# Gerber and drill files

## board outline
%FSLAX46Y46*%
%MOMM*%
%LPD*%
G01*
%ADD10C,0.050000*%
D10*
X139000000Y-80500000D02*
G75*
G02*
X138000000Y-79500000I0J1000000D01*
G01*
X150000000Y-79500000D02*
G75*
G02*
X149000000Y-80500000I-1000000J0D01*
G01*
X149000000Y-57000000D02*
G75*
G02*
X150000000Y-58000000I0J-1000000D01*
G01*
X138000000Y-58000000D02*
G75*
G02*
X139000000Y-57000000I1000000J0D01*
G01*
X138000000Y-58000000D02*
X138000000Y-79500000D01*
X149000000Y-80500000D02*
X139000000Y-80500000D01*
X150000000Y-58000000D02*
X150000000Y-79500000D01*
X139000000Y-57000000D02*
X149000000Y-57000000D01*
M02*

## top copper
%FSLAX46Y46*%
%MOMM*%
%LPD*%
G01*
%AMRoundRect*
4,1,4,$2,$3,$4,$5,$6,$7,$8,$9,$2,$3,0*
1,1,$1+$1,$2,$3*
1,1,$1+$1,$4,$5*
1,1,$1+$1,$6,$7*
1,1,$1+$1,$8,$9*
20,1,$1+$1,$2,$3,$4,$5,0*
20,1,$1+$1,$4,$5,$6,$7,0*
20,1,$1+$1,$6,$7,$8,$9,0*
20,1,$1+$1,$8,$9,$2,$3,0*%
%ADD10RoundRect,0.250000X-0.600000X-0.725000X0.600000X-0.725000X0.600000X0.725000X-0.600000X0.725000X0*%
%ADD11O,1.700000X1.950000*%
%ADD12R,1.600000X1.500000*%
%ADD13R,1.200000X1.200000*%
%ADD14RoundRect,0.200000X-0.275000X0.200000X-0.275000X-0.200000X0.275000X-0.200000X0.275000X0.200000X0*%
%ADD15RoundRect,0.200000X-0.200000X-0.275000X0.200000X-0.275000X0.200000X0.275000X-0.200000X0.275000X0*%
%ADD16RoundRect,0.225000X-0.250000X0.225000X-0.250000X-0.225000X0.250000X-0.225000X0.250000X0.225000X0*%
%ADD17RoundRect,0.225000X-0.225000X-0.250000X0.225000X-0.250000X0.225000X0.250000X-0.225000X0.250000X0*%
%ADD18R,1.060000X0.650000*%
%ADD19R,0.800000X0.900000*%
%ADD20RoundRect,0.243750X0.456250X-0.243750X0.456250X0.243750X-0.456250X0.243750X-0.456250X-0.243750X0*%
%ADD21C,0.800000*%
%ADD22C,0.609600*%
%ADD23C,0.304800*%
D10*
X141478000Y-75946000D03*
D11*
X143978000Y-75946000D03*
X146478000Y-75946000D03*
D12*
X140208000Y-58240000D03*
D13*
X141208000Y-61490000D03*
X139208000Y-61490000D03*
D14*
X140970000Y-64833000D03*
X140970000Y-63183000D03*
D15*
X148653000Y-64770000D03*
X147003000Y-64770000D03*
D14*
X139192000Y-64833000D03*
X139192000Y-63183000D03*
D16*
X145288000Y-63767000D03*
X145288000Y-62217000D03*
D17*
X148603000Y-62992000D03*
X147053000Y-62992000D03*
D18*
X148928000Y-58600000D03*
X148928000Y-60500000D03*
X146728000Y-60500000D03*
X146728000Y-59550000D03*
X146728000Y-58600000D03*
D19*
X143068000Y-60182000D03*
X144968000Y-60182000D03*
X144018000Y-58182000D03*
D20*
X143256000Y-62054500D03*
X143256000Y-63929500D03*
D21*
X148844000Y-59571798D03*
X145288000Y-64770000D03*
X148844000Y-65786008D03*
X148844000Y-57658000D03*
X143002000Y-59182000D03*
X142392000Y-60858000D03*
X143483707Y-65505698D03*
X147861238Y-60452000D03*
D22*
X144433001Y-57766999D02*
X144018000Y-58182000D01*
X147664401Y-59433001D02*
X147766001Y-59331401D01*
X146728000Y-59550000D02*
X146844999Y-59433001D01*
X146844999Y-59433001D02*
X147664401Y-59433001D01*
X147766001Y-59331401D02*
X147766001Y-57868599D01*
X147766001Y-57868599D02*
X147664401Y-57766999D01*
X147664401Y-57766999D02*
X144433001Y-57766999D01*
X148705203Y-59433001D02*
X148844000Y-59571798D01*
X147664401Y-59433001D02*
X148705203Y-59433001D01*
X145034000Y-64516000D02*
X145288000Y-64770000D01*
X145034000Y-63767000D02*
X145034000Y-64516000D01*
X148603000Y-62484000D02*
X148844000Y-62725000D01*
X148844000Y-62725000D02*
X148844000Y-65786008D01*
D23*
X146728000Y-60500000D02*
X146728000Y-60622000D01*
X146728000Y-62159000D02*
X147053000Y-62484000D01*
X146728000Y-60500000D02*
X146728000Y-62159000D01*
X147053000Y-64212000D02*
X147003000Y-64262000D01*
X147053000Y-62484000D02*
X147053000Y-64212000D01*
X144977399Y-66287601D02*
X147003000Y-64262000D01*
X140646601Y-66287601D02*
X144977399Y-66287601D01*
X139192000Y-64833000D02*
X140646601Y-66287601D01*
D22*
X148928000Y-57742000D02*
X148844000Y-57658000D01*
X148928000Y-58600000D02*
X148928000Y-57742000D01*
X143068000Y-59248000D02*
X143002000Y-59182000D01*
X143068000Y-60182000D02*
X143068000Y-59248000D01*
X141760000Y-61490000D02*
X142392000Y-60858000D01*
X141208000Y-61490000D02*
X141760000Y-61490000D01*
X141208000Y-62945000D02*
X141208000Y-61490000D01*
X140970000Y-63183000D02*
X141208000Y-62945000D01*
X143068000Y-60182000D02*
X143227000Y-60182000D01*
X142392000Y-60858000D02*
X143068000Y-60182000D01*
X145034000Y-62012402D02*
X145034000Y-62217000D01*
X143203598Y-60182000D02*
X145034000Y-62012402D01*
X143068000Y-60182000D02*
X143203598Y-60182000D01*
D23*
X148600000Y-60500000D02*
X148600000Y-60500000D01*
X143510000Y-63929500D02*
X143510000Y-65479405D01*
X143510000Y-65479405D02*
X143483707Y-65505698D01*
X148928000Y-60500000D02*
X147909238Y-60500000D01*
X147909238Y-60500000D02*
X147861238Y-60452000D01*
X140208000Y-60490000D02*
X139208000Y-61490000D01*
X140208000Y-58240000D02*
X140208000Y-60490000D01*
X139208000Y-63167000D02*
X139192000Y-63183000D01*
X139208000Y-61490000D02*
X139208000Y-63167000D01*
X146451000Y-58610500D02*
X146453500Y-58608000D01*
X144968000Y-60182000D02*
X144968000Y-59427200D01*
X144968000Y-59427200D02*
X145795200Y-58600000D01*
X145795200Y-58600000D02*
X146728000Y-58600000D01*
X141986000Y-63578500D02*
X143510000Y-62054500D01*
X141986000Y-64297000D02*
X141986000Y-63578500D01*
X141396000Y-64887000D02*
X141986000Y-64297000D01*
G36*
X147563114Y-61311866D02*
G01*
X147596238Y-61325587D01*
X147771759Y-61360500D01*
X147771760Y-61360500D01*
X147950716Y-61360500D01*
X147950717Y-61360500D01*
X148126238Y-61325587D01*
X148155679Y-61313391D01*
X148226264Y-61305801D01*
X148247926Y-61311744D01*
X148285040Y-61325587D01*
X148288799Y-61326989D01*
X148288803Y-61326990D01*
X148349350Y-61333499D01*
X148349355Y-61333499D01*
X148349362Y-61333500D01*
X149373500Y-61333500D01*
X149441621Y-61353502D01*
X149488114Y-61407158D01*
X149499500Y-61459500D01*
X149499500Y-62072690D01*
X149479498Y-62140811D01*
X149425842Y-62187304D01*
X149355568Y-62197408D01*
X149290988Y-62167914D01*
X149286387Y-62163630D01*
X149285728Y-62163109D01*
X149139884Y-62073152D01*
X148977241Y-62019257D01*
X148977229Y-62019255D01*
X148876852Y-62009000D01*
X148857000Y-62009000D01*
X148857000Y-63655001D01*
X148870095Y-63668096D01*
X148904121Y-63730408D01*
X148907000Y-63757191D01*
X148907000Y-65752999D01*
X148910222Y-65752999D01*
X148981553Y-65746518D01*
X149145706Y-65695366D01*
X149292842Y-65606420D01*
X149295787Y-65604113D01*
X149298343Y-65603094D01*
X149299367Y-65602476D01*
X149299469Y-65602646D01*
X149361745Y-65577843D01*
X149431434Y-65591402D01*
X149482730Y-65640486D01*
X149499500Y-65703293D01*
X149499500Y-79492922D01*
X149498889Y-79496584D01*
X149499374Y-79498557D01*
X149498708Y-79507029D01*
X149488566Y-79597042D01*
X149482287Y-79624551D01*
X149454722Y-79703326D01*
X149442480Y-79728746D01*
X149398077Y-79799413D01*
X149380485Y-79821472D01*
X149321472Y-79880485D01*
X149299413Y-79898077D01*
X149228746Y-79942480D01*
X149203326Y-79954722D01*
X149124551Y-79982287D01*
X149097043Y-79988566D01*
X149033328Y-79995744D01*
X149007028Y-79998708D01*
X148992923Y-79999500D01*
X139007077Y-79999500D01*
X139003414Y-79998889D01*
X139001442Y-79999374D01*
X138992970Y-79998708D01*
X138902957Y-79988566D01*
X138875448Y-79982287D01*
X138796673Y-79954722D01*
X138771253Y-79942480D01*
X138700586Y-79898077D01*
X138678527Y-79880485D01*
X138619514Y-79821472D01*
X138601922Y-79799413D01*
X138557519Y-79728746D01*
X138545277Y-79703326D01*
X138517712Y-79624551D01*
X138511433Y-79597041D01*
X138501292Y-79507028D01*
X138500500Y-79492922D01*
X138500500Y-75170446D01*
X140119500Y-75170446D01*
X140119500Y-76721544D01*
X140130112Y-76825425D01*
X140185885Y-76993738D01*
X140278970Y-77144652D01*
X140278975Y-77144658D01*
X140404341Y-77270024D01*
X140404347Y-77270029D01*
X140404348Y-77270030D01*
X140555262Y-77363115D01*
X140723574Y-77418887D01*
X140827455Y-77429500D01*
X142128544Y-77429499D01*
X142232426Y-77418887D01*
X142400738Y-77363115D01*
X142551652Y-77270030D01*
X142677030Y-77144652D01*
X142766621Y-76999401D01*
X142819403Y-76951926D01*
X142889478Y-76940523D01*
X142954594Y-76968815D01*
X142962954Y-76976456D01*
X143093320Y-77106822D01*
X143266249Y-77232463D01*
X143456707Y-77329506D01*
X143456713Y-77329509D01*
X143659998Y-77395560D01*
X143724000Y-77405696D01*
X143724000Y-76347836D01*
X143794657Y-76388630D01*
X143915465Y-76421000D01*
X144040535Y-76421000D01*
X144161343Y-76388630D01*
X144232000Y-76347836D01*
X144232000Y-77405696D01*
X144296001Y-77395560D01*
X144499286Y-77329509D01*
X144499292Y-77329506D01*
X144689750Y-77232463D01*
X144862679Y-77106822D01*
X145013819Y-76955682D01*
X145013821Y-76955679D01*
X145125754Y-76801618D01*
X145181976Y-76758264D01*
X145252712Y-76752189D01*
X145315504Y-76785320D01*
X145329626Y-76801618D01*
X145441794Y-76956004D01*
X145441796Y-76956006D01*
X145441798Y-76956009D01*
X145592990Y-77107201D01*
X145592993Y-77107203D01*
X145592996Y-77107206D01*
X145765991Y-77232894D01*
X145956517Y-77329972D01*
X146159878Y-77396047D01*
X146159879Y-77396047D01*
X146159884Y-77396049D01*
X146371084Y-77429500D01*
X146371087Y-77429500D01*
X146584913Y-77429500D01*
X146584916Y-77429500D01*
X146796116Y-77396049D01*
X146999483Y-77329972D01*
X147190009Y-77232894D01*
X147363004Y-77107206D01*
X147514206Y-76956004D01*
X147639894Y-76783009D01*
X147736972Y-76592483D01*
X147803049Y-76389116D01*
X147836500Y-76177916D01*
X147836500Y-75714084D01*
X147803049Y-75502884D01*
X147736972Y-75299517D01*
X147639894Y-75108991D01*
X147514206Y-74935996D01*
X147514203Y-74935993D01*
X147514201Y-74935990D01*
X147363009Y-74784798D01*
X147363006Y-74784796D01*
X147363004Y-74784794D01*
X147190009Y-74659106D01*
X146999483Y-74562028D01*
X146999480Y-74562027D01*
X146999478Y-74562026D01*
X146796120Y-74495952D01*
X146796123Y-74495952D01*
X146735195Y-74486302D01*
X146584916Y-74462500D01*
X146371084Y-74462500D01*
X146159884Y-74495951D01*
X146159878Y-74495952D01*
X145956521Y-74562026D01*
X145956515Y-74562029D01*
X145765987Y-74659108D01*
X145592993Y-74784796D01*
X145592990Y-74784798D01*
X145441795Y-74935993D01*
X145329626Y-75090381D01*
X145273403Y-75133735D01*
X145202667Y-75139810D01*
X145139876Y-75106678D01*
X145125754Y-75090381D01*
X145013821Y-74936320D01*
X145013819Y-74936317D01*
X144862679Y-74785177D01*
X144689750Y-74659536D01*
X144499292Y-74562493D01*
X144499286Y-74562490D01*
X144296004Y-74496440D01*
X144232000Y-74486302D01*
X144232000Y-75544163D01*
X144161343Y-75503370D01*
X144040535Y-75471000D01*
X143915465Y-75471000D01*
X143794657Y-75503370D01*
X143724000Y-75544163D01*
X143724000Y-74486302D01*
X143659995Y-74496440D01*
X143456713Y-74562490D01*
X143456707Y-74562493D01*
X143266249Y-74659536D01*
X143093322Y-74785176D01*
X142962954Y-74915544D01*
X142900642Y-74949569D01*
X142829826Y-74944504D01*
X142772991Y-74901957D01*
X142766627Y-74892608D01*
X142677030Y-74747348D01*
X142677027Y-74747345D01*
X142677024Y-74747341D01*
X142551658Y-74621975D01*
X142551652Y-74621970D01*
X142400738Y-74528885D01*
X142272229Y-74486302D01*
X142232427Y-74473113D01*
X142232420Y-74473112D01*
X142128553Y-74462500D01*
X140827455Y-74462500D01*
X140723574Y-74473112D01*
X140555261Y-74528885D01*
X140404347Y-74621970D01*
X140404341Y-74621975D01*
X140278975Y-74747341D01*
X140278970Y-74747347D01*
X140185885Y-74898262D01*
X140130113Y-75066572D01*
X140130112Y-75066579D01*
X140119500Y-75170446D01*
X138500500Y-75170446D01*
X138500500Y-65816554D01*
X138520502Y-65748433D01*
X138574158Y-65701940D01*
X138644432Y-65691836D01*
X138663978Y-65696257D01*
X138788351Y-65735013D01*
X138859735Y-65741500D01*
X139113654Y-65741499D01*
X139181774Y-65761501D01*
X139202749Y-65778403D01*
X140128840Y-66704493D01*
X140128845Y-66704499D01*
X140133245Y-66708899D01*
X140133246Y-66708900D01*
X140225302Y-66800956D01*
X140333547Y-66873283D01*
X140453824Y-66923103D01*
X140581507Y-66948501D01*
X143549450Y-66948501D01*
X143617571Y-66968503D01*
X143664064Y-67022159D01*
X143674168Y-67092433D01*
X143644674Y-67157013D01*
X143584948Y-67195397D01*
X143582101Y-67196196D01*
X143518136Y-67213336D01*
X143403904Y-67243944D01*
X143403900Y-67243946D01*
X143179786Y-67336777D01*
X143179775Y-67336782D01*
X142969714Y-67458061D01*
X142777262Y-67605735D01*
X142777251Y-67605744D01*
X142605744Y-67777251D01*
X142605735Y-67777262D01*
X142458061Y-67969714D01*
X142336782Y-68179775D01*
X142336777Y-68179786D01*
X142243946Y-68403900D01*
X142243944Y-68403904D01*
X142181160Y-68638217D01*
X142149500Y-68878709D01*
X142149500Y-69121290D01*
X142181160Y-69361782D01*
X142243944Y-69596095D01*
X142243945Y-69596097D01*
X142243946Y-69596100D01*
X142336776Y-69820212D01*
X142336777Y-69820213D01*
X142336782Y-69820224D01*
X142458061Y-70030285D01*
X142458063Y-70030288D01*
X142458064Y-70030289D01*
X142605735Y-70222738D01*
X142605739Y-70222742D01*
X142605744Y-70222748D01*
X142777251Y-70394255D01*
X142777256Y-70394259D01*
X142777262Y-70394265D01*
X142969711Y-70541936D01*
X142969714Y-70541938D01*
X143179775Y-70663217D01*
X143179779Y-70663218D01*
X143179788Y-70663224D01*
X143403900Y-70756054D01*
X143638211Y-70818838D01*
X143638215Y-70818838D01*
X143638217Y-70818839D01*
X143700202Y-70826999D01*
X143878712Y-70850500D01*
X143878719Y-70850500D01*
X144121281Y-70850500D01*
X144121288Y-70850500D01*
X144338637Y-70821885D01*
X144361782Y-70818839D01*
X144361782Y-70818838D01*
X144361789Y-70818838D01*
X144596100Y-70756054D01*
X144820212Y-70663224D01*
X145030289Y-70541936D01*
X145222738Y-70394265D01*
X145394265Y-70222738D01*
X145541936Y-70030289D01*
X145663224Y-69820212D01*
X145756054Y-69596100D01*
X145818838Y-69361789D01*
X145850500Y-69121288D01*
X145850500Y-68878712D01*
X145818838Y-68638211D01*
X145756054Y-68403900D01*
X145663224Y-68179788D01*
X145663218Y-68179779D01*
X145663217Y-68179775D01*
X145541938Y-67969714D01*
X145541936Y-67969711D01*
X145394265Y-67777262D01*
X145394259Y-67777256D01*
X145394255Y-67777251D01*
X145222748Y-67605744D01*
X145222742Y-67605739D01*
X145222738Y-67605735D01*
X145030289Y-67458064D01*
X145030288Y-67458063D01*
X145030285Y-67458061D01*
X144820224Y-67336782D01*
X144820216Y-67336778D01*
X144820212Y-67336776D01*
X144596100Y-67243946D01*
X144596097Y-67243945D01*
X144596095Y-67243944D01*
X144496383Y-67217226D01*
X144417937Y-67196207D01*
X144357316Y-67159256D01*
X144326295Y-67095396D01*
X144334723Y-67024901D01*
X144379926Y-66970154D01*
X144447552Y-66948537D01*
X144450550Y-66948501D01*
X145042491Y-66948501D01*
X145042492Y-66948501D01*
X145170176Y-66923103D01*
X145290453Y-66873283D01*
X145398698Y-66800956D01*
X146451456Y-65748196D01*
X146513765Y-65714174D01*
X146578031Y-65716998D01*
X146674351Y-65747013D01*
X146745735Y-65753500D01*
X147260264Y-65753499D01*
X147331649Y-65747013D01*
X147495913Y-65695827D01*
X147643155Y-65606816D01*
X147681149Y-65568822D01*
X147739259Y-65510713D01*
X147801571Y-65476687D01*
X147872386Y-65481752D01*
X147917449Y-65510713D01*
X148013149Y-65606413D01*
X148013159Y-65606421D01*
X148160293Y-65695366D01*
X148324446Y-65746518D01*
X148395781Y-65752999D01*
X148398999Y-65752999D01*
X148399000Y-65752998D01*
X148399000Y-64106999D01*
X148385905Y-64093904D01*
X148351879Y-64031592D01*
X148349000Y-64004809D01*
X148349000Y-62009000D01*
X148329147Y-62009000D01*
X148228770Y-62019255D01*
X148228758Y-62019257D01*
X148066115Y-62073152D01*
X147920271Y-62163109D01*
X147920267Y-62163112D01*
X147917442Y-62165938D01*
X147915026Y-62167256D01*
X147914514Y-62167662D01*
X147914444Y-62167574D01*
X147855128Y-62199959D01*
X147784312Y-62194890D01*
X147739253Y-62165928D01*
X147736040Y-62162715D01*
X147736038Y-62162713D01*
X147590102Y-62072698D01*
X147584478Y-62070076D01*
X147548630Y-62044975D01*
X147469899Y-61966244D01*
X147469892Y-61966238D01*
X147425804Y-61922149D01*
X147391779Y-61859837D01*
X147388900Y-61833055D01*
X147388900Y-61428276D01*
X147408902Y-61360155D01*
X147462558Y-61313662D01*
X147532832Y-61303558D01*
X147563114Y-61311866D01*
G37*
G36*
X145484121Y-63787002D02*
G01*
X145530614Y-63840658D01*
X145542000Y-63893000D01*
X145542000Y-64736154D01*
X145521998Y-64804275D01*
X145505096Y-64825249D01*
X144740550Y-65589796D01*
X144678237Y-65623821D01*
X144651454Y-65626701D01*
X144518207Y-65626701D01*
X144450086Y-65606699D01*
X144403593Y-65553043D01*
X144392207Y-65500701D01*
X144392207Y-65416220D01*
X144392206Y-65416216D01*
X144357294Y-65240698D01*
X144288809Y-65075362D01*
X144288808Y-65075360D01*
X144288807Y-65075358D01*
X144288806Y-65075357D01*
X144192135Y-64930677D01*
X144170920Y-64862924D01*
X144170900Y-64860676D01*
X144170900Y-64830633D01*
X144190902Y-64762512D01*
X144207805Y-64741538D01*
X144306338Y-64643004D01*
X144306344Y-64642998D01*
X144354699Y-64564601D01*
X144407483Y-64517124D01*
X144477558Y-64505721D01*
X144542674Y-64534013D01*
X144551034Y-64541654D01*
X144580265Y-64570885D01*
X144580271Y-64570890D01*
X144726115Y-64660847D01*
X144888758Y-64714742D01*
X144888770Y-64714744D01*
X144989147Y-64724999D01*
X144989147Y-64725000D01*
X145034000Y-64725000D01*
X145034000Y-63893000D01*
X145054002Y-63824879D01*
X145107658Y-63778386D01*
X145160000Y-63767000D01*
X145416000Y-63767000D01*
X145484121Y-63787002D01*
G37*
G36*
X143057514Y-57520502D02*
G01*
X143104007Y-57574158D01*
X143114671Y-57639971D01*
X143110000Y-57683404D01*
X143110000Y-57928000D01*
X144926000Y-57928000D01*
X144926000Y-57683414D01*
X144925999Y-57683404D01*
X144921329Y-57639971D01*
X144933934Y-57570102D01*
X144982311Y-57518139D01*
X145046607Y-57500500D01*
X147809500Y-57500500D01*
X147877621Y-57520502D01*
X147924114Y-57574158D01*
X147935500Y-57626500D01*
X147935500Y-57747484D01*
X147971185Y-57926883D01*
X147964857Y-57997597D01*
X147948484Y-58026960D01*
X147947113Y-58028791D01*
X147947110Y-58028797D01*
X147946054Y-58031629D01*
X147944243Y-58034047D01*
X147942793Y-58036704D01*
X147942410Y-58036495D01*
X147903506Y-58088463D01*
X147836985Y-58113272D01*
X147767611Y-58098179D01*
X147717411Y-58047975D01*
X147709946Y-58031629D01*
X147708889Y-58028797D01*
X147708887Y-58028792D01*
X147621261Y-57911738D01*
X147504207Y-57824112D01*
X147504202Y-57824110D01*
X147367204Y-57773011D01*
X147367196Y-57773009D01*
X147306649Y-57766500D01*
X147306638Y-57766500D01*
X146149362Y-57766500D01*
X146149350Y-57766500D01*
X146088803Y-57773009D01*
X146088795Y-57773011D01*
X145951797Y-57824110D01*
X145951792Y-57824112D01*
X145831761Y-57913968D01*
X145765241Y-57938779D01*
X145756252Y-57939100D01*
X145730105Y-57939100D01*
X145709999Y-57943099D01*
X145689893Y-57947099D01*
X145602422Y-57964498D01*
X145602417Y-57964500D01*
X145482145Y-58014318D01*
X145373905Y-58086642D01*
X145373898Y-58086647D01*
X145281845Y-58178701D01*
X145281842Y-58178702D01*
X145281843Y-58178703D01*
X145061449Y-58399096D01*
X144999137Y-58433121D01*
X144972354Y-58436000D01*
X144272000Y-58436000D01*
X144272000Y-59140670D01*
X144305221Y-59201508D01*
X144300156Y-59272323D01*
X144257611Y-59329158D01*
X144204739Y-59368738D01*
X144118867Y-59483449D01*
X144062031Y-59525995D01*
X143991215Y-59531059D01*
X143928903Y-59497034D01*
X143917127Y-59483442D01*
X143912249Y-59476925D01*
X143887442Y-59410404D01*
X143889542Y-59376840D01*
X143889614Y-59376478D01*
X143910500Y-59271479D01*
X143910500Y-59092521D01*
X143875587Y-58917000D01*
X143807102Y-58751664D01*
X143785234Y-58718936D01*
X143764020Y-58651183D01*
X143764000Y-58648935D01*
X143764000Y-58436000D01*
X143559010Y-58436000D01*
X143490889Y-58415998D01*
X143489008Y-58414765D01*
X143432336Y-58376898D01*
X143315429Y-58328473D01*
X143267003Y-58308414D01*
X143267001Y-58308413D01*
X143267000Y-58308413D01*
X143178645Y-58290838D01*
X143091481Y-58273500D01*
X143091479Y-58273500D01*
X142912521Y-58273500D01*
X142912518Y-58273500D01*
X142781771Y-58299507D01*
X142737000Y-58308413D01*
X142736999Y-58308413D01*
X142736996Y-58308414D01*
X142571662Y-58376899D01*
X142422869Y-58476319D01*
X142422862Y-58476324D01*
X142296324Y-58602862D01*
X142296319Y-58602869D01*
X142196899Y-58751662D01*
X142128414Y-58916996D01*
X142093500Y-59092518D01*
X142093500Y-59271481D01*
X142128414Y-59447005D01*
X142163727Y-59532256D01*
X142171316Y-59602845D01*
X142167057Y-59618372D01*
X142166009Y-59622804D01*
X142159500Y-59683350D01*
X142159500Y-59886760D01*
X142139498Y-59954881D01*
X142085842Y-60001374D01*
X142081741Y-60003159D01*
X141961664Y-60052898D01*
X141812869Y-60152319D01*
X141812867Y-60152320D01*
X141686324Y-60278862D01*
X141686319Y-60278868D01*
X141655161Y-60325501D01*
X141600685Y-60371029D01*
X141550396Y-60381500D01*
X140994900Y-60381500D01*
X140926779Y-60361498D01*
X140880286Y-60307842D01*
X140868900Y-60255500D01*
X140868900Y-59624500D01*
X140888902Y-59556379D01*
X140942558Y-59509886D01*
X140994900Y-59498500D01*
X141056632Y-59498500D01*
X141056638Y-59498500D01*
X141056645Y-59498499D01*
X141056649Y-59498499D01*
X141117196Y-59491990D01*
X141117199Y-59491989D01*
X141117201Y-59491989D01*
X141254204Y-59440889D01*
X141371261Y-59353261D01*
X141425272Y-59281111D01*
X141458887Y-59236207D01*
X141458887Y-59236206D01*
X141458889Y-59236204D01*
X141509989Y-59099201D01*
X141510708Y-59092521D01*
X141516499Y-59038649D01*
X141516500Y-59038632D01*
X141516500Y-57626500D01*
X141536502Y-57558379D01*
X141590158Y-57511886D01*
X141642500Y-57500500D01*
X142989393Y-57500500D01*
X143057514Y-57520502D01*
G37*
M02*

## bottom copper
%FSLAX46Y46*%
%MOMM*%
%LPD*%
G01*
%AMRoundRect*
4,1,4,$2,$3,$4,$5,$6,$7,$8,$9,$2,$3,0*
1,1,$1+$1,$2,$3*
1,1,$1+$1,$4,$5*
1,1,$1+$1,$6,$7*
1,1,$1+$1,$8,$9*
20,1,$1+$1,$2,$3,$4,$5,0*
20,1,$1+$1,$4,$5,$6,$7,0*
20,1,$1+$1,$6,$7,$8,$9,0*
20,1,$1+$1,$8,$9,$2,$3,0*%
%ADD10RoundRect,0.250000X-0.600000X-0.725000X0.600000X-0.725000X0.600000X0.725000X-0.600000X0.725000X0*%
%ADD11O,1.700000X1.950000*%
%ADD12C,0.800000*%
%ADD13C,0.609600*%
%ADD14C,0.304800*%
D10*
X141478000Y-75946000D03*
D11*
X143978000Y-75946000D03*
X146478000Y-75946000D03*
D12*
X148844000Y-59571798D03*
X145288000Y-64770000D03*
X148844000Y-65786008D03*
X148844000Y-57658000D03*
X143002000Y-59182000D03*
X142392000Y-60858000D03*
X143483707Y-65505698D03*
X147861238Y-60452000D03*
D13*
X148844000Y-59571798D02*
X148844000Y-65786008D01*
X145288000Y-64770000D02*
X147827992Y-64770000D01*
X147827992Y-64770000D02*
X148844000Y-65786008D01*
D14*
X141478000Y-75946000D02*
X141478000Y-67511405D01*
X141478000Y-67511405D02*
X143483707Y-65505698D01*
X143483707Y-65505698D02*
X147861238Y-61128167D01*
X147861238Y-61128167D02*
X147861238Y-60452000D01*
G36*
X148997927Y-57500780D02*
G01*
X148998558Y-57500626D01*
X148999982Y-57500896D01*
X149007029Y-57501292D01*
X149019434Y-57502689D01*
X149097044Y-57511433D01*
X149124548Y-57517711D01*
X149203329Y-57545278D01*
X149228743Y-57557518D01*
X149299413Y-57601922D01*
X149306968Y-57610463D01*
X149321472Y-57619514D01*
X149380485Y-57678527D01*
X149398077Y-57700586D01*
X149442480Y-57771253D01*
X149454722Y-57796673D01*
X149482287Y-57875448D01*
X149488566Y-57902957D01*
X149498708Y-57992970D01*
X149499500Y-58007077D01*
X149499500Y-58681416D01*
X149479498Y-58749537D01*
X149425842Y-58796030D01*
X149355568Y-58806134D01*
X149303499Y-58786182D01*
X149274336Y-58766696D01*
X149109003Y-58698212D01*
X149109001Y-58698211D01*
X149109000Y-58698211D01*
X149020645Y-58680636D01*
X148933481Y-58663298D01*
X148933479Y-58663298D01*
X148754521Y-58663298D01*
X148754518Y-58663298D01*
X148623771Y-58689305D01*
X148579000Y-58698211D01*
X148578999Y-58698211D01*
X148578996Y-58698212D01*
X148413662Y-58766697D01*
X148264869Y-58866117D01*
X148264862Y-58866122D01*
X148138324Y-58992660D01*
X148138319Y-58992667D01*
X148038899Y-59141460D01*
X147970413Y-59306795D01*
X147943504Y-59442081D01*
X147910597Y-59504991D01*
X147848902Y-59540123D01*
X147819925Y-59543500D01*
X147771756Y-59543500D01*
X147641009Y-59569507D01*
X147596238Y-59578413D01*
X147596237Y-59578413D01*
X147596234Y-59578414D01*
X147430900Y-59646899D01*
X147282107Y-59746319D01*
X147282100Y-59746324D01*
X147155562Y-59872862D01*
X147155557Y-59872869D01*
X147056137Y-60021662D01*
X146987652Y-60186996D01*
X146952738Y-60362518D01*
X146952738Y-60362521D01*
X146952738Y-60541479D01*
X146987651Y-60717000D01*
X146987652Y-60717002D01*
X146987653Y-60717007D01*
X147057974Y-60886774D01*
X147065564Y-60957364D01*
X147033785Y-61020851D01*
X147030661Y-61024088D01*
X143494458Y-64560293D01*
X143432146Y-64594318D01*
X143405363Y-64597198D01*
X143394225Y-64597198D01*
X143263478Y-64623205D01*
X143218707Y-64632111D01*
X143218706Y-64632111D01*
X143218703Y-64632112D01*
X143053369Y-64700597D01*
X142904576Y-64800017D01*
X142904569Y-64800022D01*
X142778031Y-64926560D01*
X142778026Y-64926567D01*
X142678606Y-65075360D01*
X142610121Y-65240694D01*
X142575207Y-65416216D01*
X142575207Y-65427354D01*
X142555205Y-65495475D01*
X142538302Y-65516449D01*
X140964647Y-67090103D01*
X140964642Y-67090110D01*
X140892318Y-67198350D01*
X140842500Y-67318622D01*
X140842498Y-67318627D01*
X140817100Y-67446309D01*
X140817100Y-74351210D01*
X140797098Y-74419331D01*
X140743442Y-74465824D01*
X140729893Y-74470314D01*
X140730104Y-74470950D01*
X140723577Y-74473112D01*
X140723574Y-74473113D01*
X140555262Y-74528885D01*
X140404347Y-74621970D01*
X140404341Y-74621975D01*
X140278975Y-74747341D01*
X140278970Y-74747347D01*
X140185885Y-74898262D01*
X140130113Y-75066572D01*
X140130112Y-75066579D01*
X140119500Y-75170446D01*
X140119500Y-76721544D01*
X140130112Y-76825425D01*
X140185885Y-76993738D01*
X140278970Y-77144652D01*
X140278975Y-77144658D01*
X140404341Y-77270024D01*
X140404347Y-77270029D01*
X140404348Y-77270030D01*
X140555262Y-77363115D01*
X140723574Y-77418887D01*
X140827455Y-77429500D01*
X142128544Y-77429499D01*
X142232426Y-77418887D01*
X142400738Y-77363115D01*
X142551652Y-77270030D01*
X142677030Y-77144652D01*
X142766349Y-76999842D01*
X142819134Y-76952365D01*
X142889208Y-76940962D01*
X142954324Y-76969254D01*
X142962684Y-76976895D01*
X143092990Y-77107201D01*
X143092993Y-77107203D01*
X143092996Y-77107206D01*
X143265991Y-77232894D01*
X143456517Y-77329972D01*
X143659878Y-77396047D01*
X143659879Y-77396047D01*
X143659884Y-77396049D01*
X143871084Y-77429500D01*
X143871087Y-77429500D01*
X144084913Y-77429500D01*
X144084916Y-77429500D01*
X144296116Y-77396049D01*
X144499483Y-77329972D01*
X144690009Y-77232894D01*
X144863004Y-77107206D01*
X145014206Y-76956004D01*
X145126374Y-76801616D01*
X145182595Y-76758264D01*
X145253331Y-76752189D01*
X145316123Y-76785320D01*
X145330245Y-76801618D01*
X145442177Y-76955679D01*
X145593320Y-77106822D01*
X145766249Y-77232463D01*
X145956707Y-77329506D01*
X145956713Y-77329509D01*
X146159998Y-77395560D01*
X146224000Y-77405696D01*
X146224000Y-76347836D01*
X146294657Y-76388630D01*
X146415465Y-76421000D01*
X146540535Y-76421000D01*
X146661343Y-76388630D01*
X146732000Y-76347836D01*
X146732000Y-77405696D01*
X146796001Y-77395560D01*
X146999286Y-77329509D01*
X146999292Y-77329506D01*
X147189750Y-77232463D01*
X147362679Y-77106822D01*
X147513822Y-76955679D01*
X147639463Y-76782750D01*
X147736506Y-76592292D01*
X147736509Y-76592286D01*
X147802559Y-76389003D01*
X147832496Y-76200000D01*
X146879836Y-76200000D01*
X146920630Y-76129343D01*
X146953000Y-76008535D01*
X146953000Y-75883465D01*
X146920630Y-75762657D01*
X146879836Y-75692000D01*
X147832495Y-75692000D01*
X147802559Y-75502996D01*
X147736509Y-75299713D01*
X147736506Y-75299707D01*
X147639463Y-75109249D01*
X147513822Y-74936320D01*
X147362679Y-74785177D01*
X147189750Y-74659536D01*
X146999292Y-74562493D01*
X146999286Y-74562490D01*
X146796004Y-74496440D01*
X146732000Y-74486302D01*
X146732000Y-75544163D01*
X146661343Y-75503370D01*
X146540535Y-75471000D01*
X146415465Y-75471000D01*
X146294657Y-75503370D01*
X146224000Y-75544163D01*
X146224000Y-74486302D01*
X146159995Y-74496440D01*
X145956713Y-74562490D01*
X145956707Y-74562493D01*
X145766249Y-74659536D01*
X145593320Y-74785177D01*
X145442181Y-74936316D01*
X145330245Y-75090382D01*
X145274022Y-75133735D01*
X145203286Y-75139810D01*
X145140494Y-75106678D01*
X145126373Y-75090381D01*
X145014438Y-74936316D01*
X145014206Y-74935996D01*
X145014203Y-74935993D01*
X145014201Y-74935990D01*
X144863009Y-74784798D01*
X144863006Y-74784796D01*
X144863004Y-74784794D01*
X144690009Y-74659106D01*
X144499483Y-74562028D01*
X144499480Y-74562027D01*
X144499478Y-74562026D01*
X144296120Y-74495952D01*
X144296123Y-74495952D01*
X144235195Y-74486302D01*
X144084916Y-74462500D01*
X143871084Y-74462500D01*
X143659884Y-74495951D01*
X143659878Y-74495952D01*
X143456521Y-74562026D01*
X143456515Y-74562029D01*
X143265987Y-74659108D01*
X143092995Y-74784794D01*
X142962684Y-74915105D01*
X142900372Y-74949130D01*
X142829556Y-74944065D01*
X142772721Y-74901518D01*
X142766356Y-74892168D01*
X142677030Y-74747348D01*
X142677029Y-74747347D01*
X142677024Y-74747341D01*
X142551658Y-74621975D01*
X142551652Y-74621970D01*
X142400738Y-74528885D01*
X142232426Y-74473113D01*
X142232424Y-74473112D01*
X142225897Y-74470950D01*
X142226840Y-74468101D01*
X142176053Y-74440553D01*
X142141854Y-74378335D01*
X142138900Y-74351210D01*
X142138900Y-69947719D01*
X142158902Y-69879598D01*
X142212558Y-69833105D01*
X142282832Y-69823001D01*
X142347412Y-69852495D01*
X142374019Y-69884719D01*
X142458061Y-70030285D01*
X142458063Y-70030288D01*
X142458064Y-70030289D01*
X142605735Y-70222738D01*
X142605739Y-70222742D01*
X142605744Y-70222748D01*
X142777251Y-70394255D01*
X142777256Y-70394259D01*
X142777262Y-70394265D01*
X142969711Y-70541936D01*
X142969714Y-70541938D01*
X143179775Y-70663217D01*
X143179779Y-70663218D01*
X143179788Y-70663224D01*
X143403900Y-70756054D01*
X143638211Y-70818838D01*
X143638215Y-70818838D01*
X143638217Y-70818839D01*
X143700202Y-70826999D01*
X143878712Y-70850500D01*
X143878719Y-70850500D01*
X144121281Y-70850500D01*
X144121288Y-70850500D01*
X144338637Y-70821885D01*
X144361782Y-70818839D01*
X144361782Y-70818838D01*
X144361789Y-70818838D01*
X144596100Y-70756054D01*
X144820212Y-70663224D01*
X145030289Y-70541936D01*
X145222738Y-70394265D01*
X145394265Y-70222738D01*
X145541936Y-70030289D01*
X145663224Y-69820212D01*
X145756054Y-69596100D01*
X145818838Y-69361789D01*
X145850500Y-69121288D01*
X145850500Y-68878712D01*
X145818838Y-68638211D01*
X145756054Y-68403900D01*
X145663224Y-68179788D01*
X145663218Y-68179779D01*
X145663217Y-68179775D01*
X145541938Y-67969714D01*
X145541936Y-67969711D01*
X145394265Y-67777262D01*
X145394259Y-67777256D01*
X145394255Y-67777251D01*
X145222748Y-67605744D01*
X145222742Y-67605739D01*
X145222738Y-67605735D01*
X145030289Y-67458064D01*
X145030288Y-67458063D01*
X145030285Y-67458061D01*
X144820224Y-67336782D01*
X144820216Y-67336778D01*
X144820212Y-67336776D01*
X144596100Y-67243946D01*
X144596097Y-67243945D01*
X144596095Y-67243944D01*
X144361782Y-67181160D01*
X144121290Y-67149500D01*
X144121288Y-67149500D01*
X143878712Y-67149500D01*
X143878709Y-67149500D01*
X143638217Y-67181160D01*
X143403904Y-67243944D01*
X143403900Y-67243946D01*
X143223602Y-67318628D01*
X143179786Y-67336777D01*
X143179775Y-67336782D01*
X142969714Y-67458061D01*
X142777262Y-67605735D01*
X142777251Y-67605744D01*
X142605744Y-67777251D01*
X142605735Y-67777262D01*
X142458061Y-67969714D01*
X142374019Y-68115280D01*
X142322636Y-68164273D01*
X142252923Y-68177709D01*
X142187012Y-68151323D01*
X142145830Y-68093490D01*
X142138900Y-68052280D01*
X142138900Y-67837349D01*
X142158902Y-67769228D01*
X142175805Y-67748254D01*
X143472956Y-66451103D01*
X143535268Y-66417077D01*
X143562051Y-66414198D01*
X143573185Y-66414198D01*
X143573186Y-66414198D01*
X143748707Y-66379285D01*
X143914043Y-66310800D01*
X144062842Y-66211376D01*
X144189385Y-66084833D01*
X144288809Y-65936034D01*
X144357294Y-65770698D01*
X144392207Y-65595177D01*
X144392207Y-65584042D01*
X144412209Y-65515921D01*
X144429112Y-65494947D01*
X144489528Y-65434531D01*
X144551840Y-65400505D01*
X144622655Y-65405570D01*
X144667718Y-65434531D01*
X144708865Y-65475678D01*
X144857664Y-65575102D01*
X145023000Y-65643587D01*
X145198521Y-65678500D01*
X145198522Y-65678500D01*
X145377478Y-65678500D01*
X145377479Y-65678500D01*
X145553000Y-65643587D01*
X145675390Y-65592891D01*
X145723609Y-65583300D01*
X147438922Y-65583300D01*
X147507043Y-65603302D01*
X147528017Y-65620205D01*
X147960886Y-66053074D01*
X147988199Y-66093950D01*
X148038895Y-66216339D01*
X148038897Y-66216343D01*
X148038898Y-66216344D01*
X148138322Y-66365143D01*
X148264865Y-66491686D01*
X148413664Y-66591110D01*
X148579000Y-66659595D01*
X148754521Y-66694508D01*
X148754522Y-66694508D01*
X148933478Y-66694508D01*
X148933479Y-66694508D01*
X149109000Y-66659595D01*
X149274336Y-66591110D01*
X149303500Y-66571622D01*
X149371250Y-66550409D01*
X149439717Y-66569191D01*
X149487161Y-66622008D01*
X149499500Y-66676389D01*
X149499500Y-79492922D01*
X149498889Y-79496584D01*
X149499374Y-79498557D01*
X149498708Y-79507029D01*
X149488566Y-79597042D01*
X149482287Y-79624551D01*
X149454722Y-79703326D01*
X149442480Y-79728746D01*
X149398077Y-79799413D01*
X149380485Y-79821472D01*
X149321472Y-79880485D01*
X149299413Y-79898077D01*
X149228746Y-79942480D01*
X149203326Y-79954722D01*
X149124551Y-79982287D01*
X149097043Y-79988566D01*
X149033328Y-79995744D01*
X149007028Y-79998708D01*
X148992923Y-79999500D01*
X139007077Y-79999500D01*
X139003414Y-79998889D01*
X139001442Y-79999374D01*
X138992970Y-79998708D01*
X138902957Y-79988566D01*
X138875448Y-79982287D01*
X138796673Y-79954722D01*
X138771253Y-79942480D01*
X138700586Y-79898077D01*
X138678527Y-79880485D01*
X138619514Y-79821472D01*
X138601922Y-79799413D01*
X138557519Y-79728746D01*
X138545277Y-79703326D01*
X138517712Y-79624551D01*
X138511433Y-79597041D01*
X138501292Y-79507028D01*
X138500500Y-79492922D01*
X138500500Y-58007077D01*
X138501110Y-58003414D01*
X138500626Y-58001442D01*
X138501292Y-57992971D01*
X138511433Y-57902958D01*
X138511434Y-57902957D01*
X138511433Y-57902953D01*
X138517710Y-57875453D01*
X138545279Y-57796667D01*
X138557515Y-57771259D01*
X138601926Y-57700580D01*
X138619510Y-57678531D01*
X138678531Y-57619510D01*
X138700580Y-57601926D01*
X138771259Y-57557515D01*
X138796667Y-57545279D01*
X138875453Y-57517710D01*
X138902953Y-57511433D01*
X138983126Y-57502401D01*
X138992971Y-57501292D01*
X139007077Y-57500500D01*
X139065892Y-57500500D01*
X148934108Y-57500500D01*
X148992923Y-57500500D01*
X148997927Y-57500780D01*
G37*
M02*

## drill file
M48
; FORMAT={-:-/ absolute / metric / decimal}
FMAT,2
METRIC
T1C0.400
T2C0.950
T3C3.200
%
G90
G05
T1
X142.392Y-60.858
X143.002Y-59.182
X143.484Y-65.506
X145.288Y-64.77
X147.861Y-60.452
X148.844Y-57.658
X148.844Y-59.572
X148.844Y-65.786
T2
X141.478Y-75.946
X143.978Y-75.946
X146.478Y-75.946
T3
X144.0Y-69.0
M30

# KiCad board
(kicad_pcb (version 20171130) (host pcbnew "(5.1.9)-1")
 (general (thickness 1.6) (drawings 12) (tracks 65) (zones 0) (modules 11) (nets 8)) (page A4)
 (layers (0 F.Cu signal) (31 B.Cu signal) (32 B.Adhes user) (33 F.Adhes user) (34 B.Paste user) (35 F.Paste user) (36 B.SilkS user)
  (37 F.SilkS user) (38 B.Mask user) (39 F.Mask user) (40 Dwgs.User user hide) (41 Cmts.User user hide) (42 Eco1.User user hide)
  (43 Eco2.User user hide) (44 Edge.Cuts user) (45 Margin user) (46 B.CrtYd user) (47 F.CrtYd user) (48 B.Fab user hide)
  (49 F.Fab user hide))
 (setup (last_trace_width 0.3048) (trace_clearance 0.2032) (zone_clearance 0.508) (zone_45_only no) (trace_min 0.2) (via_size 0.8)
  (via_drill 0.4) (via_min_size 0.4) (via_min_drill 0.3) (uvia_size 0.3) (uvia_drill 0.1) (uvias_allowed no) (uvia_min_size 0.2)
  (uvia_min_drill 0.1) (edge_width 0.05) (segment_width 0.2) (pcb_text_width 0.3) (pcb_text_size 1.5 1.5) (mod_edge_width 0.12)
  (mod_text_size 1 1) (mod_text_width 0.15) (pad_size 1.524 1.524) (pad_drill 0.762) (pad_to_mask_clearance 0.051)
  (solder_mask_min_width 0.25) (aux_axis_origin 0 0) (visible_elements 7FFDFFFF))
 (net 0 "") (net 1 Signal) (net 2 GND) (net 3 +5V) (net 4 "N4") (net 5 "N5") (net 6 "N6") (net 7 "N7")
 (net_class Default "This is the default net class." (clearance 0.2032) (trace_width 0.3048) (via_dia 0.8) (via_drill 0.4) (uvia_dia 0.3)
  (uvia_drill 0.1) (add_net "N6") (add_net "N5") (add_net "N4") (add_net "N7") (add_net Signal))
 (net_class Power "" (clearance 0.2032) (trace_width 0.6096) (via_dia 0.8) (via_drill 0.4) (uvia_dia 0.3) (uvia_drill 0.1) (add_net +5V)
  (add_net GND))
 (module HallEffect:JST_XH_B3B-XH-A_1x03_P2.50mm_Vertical (layer F.Cu) (at 141.478 75.946)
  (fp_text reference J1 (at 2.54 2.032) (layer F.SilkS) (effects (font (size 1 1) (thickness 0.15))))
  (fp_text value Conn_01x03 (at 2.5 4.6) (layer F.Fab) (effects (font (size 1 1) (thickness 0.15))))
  (pad 1 thru_hole roundrect (at 0 0) (size 1.7 1.95) (drill 0.95) (layers *.Cu *.Mask) (roundrect_rratio 0.147059) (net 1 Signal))
  (pad 2 thru_hole oval (at 2.5 0) (size 1.7 1.95) (drill 0.95) (layers *.Cu *.Mask) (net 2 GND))
  (pad 3 thru_hole oval (at 5 0) (size 1.7 1.95) (drill 0.95) (layers *.Cu *.Mask) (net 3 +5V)))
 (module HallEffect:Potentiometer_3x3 (layer F.Cu) (at 140.208 59.69 90)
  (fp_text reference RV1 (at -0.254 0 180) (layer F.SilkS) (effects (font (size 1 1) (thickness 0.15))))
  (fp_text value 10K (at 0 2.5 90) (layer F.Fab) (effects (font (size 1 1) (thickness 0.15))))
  (pad 2 smd rect (at 1.45 0 90) (size 1.5 1.6) (layers F.Cu F.Paste F.Mask) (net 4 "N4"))
  (pad 3 smd rect (at -1.8 1 90) (size 1.2 1.2) (layers F.Cu F.Paste F.Mask) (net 3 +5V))
  (pad 1 smd rect (at -1.8 -1 90) (size 1.2 1.2) (layers F.Cu F.Paste F.Mask) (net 4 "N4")))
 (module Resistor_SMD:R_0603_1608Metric (layer F.Cu) (at 140.97 64.008 270)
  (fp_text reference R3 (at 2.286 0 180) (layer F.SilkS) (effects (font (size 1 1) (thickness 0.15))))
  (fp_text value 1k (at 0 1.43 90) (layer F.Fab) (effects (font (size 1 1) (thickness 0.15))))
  (pad 2 smd roundrect (at 0.825 0 270) (size 0.8 0.95) (layers F.Cu F.Paste F.Mask) (roundrect_rratio 0.25) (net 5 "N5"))
  (pad 1 smd roundrect (at -0.825 0 270) (size 0.8 0.95) (layers F.Cu F.Paste F.Mask) (roundrect_rratio 0.25) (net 3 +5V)))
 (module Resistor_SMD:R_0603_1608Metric (layer F.Cu) (at 147.828 64.77)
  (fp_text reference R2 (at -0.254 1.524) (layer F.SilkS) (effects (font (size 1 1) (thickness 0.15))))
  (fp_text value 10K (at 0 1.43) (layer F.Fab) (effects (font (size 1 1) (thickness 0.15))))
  (pad 2 smd roundrect (at 0.825 0) (size 0.8 0.95) (layers F.Cu F.Paste F.Mask) (roundrect_rratio 0.25) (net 2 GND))
  (pad 1 smd roundrect (at -0.825 0) (size 0.8 0.95) (layers F.Cu F.Paste F.Mask) (roundrect_rratio 0.25) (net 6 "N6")))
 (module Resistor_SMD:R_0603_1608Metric (layer F.Cu) (at 139.192 64.008 270)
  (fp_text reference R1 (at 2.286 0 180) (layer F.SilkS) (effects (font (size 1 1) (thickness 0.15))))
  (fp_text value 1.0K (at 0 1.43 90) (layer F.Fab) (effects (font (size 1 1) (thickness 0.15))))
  (pad 2 smd roundrect (at 0.825 0 270) (size 0.8 0.95) (layers F.Cu F.Paste F.Mask) (roundrect_rratio 0.25) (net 6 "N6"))
  (pad 1 smd roundrect (at -0.825 0 270) (size 0.8 0.95) (layers F.Cu F.Paste F.Mask) (roundrect_rratio 0.25) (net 4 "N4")))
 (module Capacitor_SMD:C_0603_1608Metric (layer F.Cu) (at 145.288 62.992 270)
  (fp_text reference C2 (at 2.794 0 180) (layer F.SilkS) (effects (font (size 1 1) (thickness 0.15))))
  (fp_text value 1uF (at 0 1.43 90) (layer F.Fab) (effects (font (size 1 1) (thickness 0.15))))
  (pad 2 smd roundrect (at 0.775 0 270) (size 0.9 0.95) (layers F.Cu F.Paste F.Mask) (roundrect_rratio 0.25) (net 2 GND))
  (pad 1 smd roundrect (at -0.775 0 270) (size 0.9 0.95) (layers F.Cu F.Paste F.Mask) (roundrect_rratio 0.25) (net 3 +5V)))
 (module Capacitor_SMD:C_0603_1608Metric (layer F.Cu) (at 147.828 62.992)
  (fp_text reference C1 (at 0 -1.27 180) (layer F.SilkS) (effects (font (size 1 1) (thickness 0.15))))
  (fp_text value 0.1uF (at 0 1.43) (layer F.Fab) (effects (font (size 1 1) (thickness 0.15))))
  (pad 2 smd roundrect (at 0.775 0) (size 0.9 0.95) (layers F.Cu F.Paste F.Mask) (roundrect_rratio 0.25) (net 2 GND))
  (pad 1 smd roundrect (at -0.775 0) (size 0.9 0.95) (layers F.Cu F.Paste F.Mask) (roundrect_rratio 0.25) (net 6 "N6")))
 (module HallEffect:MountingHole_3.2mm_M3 (layer F.Cu) (at 144 69)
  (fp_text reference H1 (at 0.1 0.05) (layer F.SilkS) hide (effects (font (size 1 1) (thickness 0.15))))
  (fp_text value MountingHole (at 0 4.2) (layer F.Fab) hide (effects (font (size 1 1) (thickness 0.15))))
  (pad 1 np_thru_hole circle (at 0 0) (size 3.2 3.2) (drill 3.2) (layers *.Cu *.Mask)))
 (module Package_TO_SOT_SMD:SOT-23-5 (layer F.Cu) (at 147.828 59.55)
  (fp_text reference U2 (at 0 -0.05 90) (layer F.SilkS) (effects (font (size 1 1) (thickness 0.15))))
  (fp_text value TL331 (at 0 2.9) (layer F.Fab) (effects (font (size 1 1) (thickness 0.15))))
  (pad 5 smd rect (at 1.1 -0.95) (size 1.06 0.65) (layers F.Cu F.Paste F.Mask) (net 3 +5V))
  (pad 4 smd rect (at 1.1 0.95) (size 1.06 0.65) (layers F.Cu F.Paste F.Mask) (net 1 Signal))
  (pad 3 smd rect (at -1.1 0.95) (size 1.06 0.65) (layers F.Cu F.Paste F.Mask) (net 6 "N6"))
  (pad 2 smd rect (at -1.1 0) (size 1.06 0.65) (layers F.Cu F.Paste F.Mask) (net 2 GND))
  (pad 1 smd rect (at -1.1 -0.95) (size 1.06 0.65) (layers F.Cu F.Paste F.Mask) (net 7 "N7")))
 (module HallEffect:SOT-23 (layer F.Cu) (at 144.018 59.182 90)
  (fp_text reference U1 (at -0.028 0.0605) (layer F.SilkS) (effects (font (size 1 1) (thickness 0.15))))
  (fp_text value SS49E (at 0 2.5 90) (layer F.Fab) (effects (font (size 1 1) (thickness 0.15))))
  (pad 1 smd rect (at -1 -0.95 90) (size 0.9 0.8) (layers F.Cu F.Paste F.Mask) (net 3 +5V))
  (pad 2 smd rect (at -1 0.95 90) (size 0.9 0.8) (layers F.Cu F.Paste F.Mask) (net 7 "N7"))
  (pad 3 smd rect (at 1 0 90) (size 0.9 0.8) (layers F.Cu F.Paste F.Mask) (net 2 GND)))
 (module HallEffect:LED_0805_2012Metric (layer F.Cu) (at 143.256 62.992 90)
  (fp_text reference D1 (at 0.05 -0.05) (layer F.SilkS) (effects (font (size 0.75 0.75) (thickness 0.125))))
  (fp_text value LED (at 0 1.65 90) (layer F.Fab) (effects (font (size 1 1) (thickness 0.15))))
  (pad 2 smd roundrect (at 0.9375 0 90) (size 0.975 1.4) (layers F.Cu F.Paste F.Mask) (roundrect_rratio 0.25) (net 5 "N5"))
  (pad 1 smd roundrect (at -0.9375 0 90) (size 0.975 1.4) (layers F.Cu F.Paste F.Mask) (roundrect_rratio 0.25) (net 1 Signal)))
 (gr_arc (start 139 79.5) (end 138 79.5) (angle -90) (layer Edge.Cuts) (width 0.05))
 (gr_arc (start 149 79.5) (end 149 80.5) (angle -90) (layer Edge.Cuts) (width 0.05))
 (gr_arc (start 149 58) (end 150 58) (angle -90) (layer Edge.Cuts) (width 0.05))
 (gr_arc (start 139 58) (end 139 57) (angle -90) (layer Edge.Cuts) (width 0.05))
 (gr_line (start 138 58) (end 138 79.5) (layer Edge.Cuts) (width 0.05))
 (gr_line (start 149 80.5) (end 139 80.5) (layer Edge.Cuts) (width 0.05))
 (gr_line (start 150 58) (end 150 79.5) (layer Edge.Cuts) (width 0.05))
 (gr_line (start 139 57) (end 149 57) (layer Edge.Cuts) (width 0.05))
 (segment (start 144.433001 57.766999) (end 144.018 58.182) (width 0.6096) (layer F.Cu) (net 2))
 (segment (start 147.664401 59.433001) (end 147.766001 59.331401) (width 0.6096) (layer F.Cu) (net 2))
 (segment (start 146.728 59.55) (end 146.844999 59.433001) (width 0.6096) (layer F.Cu) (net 2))
 (segment (start 146.844999 59.433001) (end 147.664401 59.433001) (width 0.6096) (layer F.Cu) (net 2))
 (segment (start 147.766001 59.331401) (end 147.766001 57.868599) (width 0.6096) (layer F.Cu) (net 2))
 (segment (start 147.766001 57.868599) (end 147.664401 57.766999) (width 0.6096) (layer F.Cu) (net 2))
 (segment (start 147.664401 57.766999) (end 144.433001 57.766999) (width 0.6096) (layer F.Cu) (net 2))
 (via (at 148.844 59.571798) (size 0.8) (drill 0.4) (layers F.Cu B.Cu) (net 2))
 (segment (start 148.705203 59.433001) (end 148.844 59.571798) (width 0.6096) (layer F.Cu) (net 2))
 (segment (start 147.664401 59.433001) (end 148.705203 59.433001) (width 0.6096) (layer F.Cu) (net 2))
 (via (at 145.288 64.77) (size 0.8) (drill 0.4) (layers F.Cu B.Cu) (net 2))
 (segment (start 145.034 64.516) (end 145.288 64.77) (width 0.6096) (layer F.Cu) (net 2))
 (segment (start 145.034 63.767) (end 145.034 64.516) (width 0.6096) (layer F.Cu) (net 2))
 (segment (start 148.844 59.571798) (end 148.844 65.786008) (width 0.6096) (layer B.Cu) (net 2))
 (via (at 148.844 65.786008) (size 0.8) (drill 0.4) (layers F.Cu B.Cu) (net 2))
 (segment (start 148.603 62.484) (end 148.844 62.725) (width 0.6096) (layer F.Cu) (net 2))
 (segment (start 148.844 62.725) (end 148.844 65.786008) (width 0.6096) (layer F.Cu) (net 2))
 (segment (start 145.288 64.77) (end 147.827992 64.77) (width 0.6096) (layer B.Cu) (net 2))
 (segment (start 147.827992 64.77) (end 148.844 65.786008) (width 0.6096) (layer B.Cu) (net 2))
 (segment (start 146.728 60.5) (end 146.728 60.622) (width 0.3048) (layer F.Cu) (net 6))
 (segment (start 146.728 62.159) (end 147.053 62.484) (width 0.3048) (layer F.Cu) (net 6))
 (segment (start 146.728 60.5) (end 146.728 62.159) (width 0.3048) (layer F.Cu) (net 6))
 (segment (start 147.053 64.212) (end 147.003 64.262) (width 0.3048) (layer F.Cu) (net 6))
 (segment (start 147.053 62.484) (end 147.053 64.212) (width 0.3048) (layer F.Cu) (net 6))
 (segment (start 144.977399 66.287601) (end 147.003 64.262) (width 0.3048) (layer F.Cu) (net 6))
 (segment (start 140.646601 66.287601) (end 144.977399 66.287601) (width 0.3048) (layer F.Cu) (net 6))
 (segment (start 139.192 64.833) (end 140.646601 66.287601) (width 0.3048) (layer F.Cu) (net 6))
 (via (at 148.844 57.658) (size 0.8) (drill 0.4) (layers F.Cu B.Cu) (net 3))
 (segment (start 148.928 57.742) (end 148.844 57.658) (width 0.6096) (layer F.Cu) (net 3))
 (segment (start 148.928 58.6) (end 148.928 57.742) (width 0.6096) (layer F.Cu) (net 3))
 (via (at 143.002 59.182) (size 0.8) (drill 0.4) (layers F.Cu B.Cu) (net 3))
 (segment (start 143.068 59.248) (end 143.002 59.182) (width 0.6096) (layer F.Cu) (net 3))
 (segment (start 143.068 60.182) (end 143.068 59.248) (width 0.6096) (layer F.Cu) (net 3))
 (segment (start 141.76 61.49) (end 142.392 60.858) (width 0.6096) (layer F.Cu) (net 3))
 (segment (start 141.208 61.49) (end 141.76 61.49) (width 0.6096) (layer F.Cu) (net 3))
 (segment (start 141.208 62.945) (end 141.208 61.49) (width 0.6096) (layer F.Cu) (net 3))
 (segment (start 140.97 63.183) (end 141.208 62.945) (width 0.6096) (layer F.Cu) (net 3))
 (segment (start 143.068 60.182) (end 143.227 60.182) (width 0.6096) (layer F.Cu) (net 3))
 (segment (start 142.392 60.858) (end 143.068 60.182) (width 0.6096) (layer F.Cu) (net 3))
 (via (at 142.392 60.858) (size 0.8) (drill 0.4) (layers F.Cu B.Cu) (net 3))
 (segment (start 145.034 62.012402) (end 145.034 62.217) (width 0.6096) (layer F.Cu) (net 3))
 (segment (start 143.203598 60.182) (end 145.034 62.012402) (width 0.6096) (layer F.Cu) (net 3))
 (segment (start 143.068 60.182) (end 143.203598 60.182) (width 0.6096) (layer F.Cu) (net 3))
 (segment (start 148.6 60.5) (end 148.6 60.5) (width 0.3048) (layer F.Cu) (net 1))
 (segment (start 143.51 63.9295) (end 143.51 65.479405) (width 0.3048) (layer F.Cu) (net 1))
 (via (at 143.483707 65.505698) (size 0.8) (drill 0.4) (layers F.Cu B.Cu) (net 1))
 (segment (start 143.51 65.479405) (end 143.483707 65.505698) (width 0.3048) (layer F.Cu) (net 1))
 (segment (start 141.478 75.946) (end 141.478 67.511405) (width 0.3048) (layer B.Cu) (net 1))
 (segment (start 141.478 67.511405) (end 143.483707 65.505698) (width 0.3048) (layer B.Cu) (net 1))
 (segment (start 148.928 60.5) (end 147.909238 60.5) (width 0.3048) (layer F.Cu) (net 1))
 (segment (start 147.909238 60.5) (end 147.861238 60.452) (width 0.3048) (layer F.Cu) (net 1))
 (via (at 147.861238 60.452) (size 0.8) (drill 0.4) (layers F.Cu B.Cu) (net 1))
 (segment (start 143.483707 65.505698) (end 147.861238 61.128167) (width 0.3048) (layer B.Cu) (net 1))
 (segment (start 147.861238 61.128167) (end 147.861238 60.452) (width 0.3048) (layer B.Cu) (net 1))
 (segment (start 140.208 60.49) (end 139.208 61.49) (width 0.3048) (layer F.Cu) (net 4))
 (segment (start 140.208 58.24) (end 140.208 60.49) (width 0.3048) (layer F.Cu) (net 4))
 (segment (start 139.208 63.167) (end 139.192 63.183) (width 0.3048) (layer F.Cu) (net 4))
 (segment (start 139.208 61.49) (end 139.208 63.167) (width 0.3048) (layer F.Cu) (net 4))
 (segment (start 146.451 58.6105) (end 146.4535 58.608) (width 0.3048) (layer F.Cu) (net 7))
 (segment (start 144.968 60.182) (end 144.968 59.4272) (width 0.3048) (layer F.Cu) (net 7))
 (segment (start 144.968 59.4272) (end 145.7952 58.6) (width 0.3048) (layer F.Cu) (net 7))
 (segment (start 145.7952 58.6) (end 146.728 58.6) (width 0.3048) (layer F.Cu) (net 7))
 (segment (start 141.986 63.5785) (end 143.51 62.0545) (width 0.3048) (layer F.Cu) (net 5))
 (segment (start 141.986 64.297) (end 141.986 63.5785) (width 0.3048) (layer F.Cu) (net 5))
 (segment (start 141.396 64.887) (end 141.986 64.297) (width 0.3048) (layer F.Cu) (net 5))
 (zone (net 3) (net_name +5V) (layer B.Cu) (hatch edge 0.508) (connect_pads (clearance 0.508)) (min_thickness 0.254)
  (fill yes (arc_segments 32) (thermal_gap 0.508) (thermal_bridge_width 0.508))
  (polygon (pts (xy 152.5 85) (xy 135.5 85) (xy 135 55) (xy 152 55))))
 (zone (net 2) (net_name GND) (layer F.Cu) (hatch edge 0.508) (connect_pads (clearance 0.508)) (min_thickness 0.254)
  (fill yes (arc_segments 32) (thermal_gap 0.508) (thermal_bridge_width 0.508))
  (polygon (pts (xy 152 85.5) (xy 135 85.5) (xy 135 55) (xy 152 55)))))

